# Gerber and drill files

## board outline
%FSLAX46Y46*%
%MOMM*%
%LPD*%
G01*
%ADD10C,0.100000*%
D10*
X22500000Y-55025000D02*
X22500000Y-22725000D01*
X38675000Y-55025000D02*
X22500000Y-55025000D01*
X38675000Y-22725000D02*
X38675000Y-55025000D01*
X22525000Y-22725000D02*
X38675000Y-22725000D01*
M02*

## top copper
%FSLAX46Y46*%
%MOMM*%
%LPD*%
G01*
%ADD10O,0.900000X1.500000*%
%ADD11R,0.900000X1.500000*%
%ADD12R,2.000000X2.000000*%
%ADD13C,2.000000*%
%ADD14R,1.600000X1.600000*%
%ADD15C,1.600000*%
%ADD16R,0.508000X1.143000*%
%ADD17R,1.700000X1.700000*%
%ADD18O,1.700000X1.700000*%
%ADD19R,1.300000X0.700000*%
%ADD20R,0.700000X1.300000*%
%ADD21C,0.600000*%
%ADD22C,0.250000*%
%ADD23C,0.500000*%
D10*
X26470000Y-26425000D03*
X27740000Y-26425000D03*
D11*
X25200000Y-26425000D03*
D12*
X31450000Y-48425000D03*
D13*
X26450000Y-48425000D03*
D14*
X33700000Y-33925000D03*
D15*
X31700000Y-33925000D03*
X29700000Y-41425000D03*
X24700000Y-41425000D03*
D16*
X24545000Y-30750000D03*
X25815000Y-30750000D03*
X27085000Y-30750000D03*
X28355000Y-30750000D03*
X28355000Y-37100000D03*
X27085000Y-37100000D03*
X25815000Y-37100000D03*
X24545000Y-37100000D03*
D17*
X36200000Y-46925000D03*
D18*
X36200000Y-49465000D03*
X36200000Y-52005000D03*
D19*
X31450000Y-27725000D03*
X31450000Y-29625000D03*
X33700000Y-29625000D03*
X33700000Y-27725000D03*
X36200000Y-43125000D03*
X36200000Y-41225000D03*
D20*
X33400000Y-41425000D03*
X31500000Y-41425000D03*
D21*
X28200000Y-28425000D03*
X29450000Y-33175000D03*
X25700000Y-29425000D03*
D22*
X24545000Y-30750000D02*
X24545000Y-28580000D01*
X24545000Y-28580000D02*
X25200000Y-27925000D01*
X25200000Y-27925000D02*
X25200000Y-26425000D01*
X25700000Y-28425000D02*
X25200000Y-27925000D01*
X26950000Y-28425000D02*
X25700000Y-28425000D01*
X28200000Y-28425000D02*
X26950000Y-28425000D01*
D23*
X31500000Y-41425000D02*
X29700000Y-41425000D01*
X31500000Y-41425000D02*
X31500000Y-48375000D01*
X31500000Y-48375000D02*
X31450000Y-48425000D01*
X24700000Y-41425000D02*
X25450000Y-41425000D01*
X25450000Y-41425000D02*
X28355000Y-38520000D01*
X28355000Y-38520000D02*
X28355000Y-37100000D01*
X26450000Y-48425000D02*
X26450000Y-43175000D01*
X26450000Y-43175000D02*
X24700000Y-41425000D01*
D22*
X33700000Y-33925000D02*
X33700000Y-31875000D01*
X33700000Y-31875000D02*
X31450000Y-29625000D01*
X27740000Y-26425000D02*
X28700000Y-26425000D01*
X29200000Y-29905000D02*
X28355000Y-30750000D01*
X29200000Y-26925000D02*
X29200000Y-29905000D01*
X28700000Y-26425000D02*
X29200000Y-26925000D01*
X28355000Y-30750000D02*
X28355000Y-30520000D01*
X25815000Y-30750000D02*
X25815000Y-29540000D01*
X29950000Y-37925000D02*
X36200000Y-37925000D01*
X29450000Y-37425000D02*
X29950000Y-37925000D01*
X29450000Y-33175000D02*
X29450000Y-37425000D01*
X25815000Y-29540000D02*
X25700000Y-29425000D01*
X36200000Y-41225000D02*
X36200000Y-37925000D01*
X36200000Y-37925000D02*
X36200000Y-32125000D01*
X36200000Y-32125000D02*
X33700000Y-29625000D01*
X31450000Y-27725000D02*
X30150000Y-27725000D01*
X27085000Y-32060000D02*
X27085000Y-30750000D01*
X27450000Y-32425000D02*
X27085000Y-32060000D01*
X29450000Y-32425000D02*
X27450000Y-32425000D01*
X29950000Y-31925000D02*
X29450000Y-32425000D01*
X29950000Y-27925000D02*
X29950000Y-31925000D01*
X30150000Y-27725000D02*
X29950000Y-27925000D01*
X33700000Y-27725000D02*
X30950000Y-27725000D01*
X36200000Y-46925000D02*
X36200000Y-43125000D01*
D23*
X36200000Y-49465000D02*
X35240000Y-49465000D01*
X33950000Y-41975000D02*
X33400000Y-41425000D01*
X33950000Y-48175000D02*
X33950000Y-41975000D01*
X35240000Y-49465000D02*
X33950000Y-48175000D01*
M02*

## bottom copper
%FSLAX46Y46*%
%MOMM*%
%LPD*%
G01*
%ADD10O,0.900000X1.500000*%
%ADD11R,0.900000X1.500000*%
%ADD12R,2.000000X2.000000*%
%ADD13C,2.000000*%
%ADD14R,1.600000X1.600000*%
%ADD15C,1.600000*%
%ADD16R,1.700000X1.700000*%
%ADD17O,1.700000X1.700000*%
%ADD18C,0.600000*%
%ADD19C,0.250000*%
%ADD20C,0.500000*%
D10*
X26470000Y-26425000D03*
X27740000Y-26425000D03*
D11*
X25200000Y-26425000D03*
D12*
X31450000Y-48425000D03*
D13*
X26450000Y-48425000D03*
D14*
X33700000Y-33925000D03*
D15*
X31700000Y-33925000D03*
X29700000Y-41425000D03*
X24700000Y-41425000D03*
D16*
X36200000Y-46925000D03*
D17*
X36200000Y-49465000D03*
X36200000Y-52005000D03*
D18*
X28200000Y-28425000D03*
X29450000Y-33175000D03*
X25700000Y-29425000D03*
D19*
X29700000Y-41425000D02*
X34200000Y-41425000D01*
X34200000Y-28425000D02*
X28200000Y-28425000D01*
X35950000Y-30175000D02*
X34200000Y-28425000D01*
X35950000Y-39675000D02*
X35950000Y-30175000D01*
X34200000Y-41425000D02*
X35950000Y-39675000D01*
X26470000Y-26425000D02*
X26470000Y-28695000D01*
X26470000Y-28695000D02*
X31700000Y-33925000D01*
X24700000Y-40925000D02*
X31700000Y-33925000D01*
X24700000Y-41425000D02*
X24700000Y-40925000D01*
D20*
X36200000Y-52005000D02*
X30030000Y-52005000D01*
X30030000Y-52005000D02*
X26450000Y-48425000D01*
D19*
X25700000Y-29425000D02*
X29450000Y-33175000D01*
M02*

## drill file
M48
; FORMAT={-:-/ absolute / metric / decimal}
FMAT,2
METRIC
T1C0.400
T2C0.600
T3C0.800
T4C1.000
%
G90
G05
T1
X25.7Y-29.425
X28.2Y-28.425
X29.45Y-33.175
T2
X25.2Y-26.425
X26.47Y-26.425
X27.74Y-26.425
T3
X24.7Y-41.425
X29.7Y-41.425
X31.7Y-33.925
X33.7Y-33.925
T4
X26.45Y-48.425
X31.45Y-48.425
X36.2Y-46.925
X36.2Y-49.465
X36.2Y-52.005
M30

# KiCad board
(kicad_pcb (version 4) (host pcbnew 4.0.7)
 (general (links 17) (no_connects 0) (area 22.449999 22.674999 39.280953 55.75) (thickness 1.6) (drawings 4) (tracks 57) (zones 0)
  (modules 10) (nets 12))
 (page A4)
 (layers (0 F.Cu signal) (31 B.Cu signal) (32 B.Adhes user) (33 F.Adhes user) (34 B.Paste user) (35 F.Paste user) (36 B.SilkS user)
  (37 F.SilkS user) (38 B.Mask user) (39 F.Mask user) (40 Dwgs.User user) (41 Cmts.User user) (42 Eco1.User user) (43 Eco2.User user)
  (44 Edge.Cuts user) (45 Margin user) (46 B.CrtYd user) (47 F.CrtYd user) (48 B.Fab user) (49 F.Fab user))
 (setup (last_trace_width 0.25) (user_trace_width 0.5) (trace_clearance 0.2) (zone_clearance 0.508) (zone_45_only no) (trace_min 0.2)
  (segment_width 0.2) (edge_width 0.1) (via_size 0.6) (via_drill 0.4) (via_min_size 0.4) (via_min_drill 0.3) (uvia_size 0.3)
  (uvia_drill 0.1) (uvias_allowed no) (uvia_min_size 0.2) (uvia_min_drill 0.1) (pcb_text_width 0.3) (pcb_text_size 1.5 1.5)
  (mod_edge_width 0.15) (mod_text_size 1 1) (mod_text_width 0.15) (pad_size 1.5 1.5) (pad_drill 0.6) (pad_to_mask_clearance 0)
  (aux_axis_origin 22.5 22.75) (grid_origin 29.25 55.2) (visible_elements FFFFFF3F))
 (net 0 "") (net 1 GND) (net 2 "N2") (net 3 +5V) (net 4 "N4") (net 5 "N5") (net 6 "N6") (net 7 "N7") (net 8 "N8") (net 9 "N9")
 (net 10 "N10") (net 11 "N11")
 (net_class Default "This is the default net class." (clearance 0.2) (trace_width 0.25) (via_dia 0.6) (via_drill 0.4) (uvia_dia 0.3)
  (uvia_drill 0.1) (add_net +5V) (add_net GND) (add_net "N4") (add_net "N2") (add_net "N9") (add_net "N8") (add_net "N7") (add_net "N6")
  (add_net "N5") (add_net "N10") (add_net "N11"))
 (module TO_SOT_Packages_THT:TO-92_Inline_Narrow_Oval (layer F.Cu) (at 25.2 26.425)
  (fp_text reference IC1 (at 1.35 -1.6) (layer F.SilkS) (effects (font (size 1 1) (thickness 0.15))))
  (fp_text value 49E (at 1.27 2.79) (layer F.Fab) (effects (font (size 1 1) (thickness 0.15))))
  (pad 2 thru_hole oval (at 1.27 0 180) (size 0.9 1.5) (drill 0.6) (layers *.Cu *.Mask) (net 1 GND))
  (pad 3 thru_hole oval (at 2.54 0 180) (size 0.9 1.5) (drill 0.6) (layers *.Cu *.Mask) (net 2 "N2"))
  (pad 1 thru_hole rect (at 0 0 180) (size 0.9 1.5) (drill 0.6) (layers *.Cu *.Mask) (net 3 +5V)))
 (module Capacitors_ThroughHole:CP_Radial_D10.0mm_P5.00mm (layer F.Cu) (at 31.45 48.425 180)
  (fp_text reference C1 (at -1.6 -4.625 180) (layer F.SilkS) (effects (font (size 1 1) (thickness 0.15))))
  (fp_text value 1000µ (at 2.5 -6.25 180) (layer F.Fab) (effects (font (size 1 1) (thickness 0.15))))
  (pad 1 thru_hole rect (at 0 0 180) (size 2 2) (drill 1) (layers *.Cu *.Mask) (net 3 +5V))
  (pad 2 thru_hole circle (at 5 0 180) (size 2 2) (drill 1) (layers *.Cu *.Mask) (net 1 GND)))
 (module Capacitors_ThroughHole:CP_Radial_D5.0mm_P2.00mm (layer F.Cu) (at 33.7 33.925 180)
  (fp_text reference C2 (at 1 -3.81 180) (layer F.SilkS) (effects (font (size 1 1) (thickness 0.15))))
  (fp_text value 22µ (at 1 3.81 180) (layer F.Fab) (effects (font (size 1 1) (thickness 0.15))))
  (pad 1 thru_hole rect (at 0 0 180) (size 1.6 1.6) (drill 0.8) (layers *.Cu *.Mask) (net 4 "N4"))
  (pad 2 thru_hole circle (at 2 0 180) (size 1.6 1.6) (drill 0.8) (layers *.Cu *.Mask) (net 1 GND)))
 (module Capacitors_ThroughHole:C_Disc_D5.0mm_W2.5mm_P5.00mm (layer F.Cu) (at 29.7 41.425 180)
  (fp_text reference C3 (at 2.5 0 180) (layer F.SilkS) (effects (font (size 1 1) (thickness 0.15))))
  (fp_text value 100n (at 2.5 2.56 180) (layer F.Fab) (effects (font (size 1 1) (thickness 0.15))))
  (pad 1 thru_hole circle (at 0 0 180) (size 1.6 1.6) (drill 0.8) (layers *.Cu *.Mask) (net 3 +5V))
  (pad 2 thru_hole circle (at 5 0 180) (size 1.6 1.6) (drill 0.8) (layers *.Cu *.Mask) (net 1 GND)))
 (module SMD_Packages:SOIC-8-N (layer F.Cu) (at 26.45 33.925)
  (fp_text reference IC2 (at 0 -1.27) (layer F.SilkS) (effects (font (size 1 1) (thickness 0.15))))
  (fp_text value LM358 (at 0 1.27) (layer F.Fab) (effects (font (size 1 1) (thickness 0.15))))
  (pad 8 smd rect (at -1.905 -3.175) (size 0.508 1.143) (layers F.Cu F.Paste F.Mask) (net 3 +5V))
  (pad 7 smd rect (at -0.635 -3.175) (size 0.508 1.143) (layers F.Cu F.Paste F.Mask) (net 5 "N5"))
  (pad 6 smd rect (at 0.635 -3.175) (size 0.508 1.143) (layers F.Cu F.Paste F.Mask) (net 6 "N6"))
  (pad 5 smd rect (at 1.905 -3.175) (size 0.508 1.143) (layers F.Cu F.Paste F.Mask) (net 2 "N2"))
  (pad 4 smd rect (at 1.905 3.175) (size 0.508 1.143) (layers F.Cu F.Paste F.Mask) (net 1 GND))
  (pad 3 smd rect (at 0.635 3.175) (size 0.508 1.143) (layers F.Cu F.Paste F.Mask) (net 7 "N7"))
  (pad 2 smd rect (at -0.635 3.175) (size 0.508 1.143) (layers F.Cu F.Paste F.Mask) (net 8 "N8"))
  (pad 1 smd rect (at -1.905 3.175) (size 0.508 1.143) (layers F.Cu F.Paste F.Mask) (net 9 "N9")))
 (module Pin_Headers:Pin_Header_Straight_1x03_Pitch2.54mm (layer F.Cu) (at 36.2 46.925)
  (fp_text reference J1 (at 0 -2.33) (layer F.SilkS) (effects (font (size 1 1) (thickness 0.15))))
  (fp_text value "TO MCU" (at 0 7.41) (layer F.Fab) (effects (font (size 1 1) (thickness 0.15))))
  (pad 1 thru_hole rect (at 0 0) (size 1.7 1.7) (drill 1) (layers *.Cu *.Mask) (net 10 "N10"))
  (pad 2 thru_hole oval (at 0 2.54) (size 1.7 1.7) (drill 1) (layers *.Cu *.Mask) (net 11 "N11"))
  (pad 3 thru_hole oval (at 0 5.08) (size 1.7 1.7) (drill 1) (layers *.Cu *.Mask) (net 1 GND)))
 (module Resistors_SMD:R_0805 (layer F.Cu) (at 31.45 28.675 270)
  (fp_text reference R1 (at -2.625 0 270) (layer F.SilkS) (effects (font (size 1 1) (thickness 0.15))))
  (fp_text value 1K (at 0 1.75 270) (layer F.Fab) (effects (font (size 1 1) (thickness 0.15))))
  (pad 1 smd rect (at -0.95 0 270) (size 0.7 1.3) (layers F.Cu F.Paste F.Mask) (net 6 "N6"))
  (pad 2 smd rect (at 0.95 0 270) (size 0.7 1.3) (layers F.Cu F.Paste F.Mask) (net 4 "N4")))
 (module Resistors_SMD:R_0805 (layer F.Cu) (at 33.7 28.675 90)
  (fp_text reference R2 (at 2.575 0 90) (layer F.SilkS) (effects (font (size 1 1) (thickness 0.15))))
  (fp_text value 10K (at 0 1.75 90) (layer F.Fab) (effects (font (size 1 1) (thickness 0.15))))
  (pad 1 smd rect (at -0.95 0 90) (size 0.7 1.3) (layers F.Cu F.Paste F.Mask) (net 5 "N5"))
  (pad 2 smd rect (at 0.95 0 90) (size 0.7 1.3) (layers F.Cu F.Paste F.Mask) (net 6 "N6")))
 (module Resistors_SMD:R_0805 (layer F.Cu) (at 36.2 42.175 90)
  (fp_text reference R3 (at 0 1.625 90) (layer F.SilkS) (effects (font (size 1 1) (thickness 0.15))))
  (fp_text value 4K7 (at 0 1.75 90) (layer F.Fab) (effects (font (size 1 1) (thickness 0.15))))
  (pad 1 smd rect (at -0.95 0 90) (size 0.7 1.3) (layers F.Cu F.Paste F.Mask) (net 10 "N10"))
  (pad 2 smd rect (at 0.95 0 90) (size 0.7 1.3) (layers F.Cu F.Paste F.Mask) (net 5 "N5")))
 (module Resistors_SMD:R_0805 (layer F.Cu) (at 32.45 41.425 180)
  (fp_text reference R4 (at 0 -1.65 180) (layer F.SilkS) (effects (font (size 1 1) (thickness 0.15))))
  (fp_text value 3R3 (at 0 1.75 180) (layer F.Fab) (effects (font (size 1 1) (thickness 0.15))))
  (pad 1 smd rect (at -0.95 0 180) (size 0.7 1.3) (layers F.Cu F.Paste F.Mask) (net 11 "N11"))
  (pad 2 smd rect (at 0.95 0 180) (size 0.7 1.3) (layers F.Cu F.Paste F.Mask) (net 3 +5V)))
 (gr_line (start 22.5 55.025) (end 22.5 22.725) (angle 90) (layer Edge.Cuts) (width 0.1))
 (gr_line (start 38.675 55.025) (end 22.5 55.025) (angle 90) (layer Edge.Cuts) (width 0.1))
 (gr_line (start 38.675 22.725) (end 38.675 55.025) (angle 90) (layer Edge.Cuts) (width 0.1))
 (gr_line (start 22.525 22.725) (end 38.675 22.725) (angle 90) (layer Edge.Cuts) (width 0.1))
 (segment (start 24.545 30.75) (end 24.545 28.58) (width 0.25) (layer F.Cu) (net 3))
 (segment (start 24.545 28.58) (end 25.2 27.925) (width 0.25) (layer F.Cu) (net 3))
 (segment (start 29.7 41.425) (end 34.2 41.425) (width 0.25) (layer B.Cu) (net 3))
 (segment (start 25.2 27.925) (end 25.2 26.425) (width 0.25) (layer F.Cu) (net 3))
 (segment (start 25.7 28.425) (end 25.2 27.925) (width 0.25) (layer F.Cu) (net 3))
 (segment (start 26.95 28.425) (end 25.7 28.425) (width 0.25) (layer F.Cu) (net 3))
 (segment (start 28.2 28.425) (end 26.95 28.425) (width 0.25) (layer F.Cu) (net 3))
 (via (at 28.2 28.425) (size 0.6) (drill 0.4) (layers F.Cu B.Cu) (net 3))
 (segment (start 34.2 28.425) (end 28.2 28.425) (width 0.25) (layer B.Cu) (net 3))
 (segment (start 35.95 30.175) (end 34.2 28.425) (width 0.25) (layer B.Cu) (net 3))
 (segment (start 35.95 39.675) (end 35.95 30.175) (width 0.25) (layer B.Cu) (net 3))
 (segment (start 34.2 41.425) (end 35.95 39.675) (width 0.25) (layer B.Cu) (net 3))
 (segment (start 31.5 41.425) (end 29.7 41.425) (width 0.5) (layer F.Cu) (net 3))
 (segment (start 31.5 41.425) (end 31.5 48.375) (width 0.5) (layer F.Cu) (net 3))
 (segment (start 31.5 48.375) (end 31.45 48.425) (width 0.5) (layer F.Cu) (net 3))
 (segment (start 26.47 26.425) (end 26.47 28.695) (width 0.25) (layer B.Cu) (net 1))
 (segment (start 26.47 28.695) (end 31.7 33.925) (width 0.25) (layer B.Cu) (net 1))
 (segment (start 24.7 40.925) (end 31.7 33.925) (width 0.25) (layer B.Cu) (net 1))
 (segment (start 24.7 41.425) (end 24.7 40.925) (width 0.25) (layer B.Cu) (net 1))
 (segment (start 36.2 52.005) (end 30.03 52.005) (width 0.5) (layer B.Cu) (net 1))
 (segment (start 30.03 52.005) (end 26.45 48.425) (width 0.5) (layer B.Cu) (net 1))
 (segment (start 24.7 41.425) (end 25.45 41.425) (width 0.5) (layer F.Cu) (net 1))
 (segment (start 25.45 41.425) (end 28.355 38.52) (width 0.5) (layer F.Cu) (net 1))
 (segment (start 28.355 38.52) (end 28.355 37.1) (width 0.5) (layer F.Cu) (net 1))
 (segment (start 26.45 48.425) (end 26.45 43.175) (width 0.5) (layer F.Cu) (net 1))
 (segment (start 26.45 43.175) (end 24.7 41.425) (width 0.5) (layer F.Cu) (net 1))
 (segment (start 33.7 33.925) (end 33.7 31.875) (width 0.25) (layer F.Cu) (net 4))
 (segment (start 33.7 31.875) (end 31.45 29.625) (width 0.25) (layer F.Cu) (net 4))
 (segment (start 27.74 26.425) (end 28.7 26.425) (width 0.25) (layer F.Cu) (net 2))
 (segment (start 29.2 29.905) (end 28.355 30.75) (width 0.25) (layer F.Cu) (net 2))
 (segment (start 29.2 26.925) (end 29.2 29.905) (width 0.25) (layer F.Cu) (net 2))
 (segment (start 28.7 26.425) (end 29.2 26.925) (width 0.25) (layer F.Cu) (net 2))
 (segment (start 28.355 30.75) (end 28.355 30.52) (width 0.25) (layer F.Cu) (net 2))
 (segment (start 25.815 30.75) (end 25.815 29.54) (width 0.25) (layer F.Cu) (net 5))
 (segment (start 29.95 37.925) (end 36.2 37.925) (width 0.25) (layer F.Cu) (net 5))
 (segment (start 29.45 37.425) (end 29.95 37.925) (width 0.25) (layer F.Cu) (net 5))
 (segment (start 29.45 33.175) (end 29.45 37.425) (width 0.25) (layer F.Cu) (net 5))
 (via (at 29.45 33.175) (size 0.6) (drill 0.4) (layers F.Cu B.Cu) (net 5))
 (segment (start 25.7 29.425) (end 29.45 33.175) (width 0.25) (layer B.Cu) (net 5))
 (via (at 25.7 29.425) (size 0.6) (drill 0.4) (layers F.Cu B.Cu) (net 5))
 (segment (start 25.815 29.54) (end 25.7 29.425) (width 0.25) (layer F.Cu) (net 5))
 (segment (start 36.2 41.225) (end 36.2 37.925) (width 0.25) (layer F.Cu) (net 5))
 (segment (start 36.2 37.925) (end 36.2 32.125) (width 0.25) (layer F.Cu) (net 5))
 (segment (start 36.2 32.125) (end 33.7 29.625) (width 0.25) (layer F.Cu) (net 5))
 (segment (start 31.45 27.725) (end 30.15 27.725) (width 0.25) (layer F.Cu) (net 6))
 (segment (start 27.085 32.06) (end 27.085 30.75) (width 0.25) (layer F.Cu) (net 6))
 (segment (start 27.45 32.425) (end 27.085 32.06) (width 0.25) (layer F.Cu) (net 6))
 (segment (start 29.45 32.425) (end 27.45 32.425) (width 0.25) (layer F.Cu) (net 6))
 (segment (start 29.95 31.925) (end 29.45 32.425) (width 0.25) (layer F.Cu) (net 6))
 (segment (start 29.95 27.925) (end 29.95 31.925) (width 0.25) (layer F.Cu) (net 6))
 (segment (start 30.15 27.725) (end 29.95 27.925) (width 0.25) (layer F.Cu) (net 6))
 (segment (start 33.7 27.725) (end 30.95 27.725) (width 0.25) (layer F.Cu) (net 6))
 (segment (start 36.2 46.925) (end 36.2 43.125) (width 0.25) (layer F.Cu) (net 10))
 (segment (start 36.2 49.465) (end 35.24 49.465) (width 0.5) (layer F.Cu) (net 11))
 (segment (start 33.95 41.975) (end 33.4 41.425) (width 0.5) (layer F.Cu) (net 11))
 (segment (start 33.95 48.175) (end 33.95 41.975) (width 0.5) (layer F.Cu) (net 11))
 (segment (start 35.24 49.465) (end 33.95 48.175) (width 0.5) (layer F.Cu) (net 11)))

